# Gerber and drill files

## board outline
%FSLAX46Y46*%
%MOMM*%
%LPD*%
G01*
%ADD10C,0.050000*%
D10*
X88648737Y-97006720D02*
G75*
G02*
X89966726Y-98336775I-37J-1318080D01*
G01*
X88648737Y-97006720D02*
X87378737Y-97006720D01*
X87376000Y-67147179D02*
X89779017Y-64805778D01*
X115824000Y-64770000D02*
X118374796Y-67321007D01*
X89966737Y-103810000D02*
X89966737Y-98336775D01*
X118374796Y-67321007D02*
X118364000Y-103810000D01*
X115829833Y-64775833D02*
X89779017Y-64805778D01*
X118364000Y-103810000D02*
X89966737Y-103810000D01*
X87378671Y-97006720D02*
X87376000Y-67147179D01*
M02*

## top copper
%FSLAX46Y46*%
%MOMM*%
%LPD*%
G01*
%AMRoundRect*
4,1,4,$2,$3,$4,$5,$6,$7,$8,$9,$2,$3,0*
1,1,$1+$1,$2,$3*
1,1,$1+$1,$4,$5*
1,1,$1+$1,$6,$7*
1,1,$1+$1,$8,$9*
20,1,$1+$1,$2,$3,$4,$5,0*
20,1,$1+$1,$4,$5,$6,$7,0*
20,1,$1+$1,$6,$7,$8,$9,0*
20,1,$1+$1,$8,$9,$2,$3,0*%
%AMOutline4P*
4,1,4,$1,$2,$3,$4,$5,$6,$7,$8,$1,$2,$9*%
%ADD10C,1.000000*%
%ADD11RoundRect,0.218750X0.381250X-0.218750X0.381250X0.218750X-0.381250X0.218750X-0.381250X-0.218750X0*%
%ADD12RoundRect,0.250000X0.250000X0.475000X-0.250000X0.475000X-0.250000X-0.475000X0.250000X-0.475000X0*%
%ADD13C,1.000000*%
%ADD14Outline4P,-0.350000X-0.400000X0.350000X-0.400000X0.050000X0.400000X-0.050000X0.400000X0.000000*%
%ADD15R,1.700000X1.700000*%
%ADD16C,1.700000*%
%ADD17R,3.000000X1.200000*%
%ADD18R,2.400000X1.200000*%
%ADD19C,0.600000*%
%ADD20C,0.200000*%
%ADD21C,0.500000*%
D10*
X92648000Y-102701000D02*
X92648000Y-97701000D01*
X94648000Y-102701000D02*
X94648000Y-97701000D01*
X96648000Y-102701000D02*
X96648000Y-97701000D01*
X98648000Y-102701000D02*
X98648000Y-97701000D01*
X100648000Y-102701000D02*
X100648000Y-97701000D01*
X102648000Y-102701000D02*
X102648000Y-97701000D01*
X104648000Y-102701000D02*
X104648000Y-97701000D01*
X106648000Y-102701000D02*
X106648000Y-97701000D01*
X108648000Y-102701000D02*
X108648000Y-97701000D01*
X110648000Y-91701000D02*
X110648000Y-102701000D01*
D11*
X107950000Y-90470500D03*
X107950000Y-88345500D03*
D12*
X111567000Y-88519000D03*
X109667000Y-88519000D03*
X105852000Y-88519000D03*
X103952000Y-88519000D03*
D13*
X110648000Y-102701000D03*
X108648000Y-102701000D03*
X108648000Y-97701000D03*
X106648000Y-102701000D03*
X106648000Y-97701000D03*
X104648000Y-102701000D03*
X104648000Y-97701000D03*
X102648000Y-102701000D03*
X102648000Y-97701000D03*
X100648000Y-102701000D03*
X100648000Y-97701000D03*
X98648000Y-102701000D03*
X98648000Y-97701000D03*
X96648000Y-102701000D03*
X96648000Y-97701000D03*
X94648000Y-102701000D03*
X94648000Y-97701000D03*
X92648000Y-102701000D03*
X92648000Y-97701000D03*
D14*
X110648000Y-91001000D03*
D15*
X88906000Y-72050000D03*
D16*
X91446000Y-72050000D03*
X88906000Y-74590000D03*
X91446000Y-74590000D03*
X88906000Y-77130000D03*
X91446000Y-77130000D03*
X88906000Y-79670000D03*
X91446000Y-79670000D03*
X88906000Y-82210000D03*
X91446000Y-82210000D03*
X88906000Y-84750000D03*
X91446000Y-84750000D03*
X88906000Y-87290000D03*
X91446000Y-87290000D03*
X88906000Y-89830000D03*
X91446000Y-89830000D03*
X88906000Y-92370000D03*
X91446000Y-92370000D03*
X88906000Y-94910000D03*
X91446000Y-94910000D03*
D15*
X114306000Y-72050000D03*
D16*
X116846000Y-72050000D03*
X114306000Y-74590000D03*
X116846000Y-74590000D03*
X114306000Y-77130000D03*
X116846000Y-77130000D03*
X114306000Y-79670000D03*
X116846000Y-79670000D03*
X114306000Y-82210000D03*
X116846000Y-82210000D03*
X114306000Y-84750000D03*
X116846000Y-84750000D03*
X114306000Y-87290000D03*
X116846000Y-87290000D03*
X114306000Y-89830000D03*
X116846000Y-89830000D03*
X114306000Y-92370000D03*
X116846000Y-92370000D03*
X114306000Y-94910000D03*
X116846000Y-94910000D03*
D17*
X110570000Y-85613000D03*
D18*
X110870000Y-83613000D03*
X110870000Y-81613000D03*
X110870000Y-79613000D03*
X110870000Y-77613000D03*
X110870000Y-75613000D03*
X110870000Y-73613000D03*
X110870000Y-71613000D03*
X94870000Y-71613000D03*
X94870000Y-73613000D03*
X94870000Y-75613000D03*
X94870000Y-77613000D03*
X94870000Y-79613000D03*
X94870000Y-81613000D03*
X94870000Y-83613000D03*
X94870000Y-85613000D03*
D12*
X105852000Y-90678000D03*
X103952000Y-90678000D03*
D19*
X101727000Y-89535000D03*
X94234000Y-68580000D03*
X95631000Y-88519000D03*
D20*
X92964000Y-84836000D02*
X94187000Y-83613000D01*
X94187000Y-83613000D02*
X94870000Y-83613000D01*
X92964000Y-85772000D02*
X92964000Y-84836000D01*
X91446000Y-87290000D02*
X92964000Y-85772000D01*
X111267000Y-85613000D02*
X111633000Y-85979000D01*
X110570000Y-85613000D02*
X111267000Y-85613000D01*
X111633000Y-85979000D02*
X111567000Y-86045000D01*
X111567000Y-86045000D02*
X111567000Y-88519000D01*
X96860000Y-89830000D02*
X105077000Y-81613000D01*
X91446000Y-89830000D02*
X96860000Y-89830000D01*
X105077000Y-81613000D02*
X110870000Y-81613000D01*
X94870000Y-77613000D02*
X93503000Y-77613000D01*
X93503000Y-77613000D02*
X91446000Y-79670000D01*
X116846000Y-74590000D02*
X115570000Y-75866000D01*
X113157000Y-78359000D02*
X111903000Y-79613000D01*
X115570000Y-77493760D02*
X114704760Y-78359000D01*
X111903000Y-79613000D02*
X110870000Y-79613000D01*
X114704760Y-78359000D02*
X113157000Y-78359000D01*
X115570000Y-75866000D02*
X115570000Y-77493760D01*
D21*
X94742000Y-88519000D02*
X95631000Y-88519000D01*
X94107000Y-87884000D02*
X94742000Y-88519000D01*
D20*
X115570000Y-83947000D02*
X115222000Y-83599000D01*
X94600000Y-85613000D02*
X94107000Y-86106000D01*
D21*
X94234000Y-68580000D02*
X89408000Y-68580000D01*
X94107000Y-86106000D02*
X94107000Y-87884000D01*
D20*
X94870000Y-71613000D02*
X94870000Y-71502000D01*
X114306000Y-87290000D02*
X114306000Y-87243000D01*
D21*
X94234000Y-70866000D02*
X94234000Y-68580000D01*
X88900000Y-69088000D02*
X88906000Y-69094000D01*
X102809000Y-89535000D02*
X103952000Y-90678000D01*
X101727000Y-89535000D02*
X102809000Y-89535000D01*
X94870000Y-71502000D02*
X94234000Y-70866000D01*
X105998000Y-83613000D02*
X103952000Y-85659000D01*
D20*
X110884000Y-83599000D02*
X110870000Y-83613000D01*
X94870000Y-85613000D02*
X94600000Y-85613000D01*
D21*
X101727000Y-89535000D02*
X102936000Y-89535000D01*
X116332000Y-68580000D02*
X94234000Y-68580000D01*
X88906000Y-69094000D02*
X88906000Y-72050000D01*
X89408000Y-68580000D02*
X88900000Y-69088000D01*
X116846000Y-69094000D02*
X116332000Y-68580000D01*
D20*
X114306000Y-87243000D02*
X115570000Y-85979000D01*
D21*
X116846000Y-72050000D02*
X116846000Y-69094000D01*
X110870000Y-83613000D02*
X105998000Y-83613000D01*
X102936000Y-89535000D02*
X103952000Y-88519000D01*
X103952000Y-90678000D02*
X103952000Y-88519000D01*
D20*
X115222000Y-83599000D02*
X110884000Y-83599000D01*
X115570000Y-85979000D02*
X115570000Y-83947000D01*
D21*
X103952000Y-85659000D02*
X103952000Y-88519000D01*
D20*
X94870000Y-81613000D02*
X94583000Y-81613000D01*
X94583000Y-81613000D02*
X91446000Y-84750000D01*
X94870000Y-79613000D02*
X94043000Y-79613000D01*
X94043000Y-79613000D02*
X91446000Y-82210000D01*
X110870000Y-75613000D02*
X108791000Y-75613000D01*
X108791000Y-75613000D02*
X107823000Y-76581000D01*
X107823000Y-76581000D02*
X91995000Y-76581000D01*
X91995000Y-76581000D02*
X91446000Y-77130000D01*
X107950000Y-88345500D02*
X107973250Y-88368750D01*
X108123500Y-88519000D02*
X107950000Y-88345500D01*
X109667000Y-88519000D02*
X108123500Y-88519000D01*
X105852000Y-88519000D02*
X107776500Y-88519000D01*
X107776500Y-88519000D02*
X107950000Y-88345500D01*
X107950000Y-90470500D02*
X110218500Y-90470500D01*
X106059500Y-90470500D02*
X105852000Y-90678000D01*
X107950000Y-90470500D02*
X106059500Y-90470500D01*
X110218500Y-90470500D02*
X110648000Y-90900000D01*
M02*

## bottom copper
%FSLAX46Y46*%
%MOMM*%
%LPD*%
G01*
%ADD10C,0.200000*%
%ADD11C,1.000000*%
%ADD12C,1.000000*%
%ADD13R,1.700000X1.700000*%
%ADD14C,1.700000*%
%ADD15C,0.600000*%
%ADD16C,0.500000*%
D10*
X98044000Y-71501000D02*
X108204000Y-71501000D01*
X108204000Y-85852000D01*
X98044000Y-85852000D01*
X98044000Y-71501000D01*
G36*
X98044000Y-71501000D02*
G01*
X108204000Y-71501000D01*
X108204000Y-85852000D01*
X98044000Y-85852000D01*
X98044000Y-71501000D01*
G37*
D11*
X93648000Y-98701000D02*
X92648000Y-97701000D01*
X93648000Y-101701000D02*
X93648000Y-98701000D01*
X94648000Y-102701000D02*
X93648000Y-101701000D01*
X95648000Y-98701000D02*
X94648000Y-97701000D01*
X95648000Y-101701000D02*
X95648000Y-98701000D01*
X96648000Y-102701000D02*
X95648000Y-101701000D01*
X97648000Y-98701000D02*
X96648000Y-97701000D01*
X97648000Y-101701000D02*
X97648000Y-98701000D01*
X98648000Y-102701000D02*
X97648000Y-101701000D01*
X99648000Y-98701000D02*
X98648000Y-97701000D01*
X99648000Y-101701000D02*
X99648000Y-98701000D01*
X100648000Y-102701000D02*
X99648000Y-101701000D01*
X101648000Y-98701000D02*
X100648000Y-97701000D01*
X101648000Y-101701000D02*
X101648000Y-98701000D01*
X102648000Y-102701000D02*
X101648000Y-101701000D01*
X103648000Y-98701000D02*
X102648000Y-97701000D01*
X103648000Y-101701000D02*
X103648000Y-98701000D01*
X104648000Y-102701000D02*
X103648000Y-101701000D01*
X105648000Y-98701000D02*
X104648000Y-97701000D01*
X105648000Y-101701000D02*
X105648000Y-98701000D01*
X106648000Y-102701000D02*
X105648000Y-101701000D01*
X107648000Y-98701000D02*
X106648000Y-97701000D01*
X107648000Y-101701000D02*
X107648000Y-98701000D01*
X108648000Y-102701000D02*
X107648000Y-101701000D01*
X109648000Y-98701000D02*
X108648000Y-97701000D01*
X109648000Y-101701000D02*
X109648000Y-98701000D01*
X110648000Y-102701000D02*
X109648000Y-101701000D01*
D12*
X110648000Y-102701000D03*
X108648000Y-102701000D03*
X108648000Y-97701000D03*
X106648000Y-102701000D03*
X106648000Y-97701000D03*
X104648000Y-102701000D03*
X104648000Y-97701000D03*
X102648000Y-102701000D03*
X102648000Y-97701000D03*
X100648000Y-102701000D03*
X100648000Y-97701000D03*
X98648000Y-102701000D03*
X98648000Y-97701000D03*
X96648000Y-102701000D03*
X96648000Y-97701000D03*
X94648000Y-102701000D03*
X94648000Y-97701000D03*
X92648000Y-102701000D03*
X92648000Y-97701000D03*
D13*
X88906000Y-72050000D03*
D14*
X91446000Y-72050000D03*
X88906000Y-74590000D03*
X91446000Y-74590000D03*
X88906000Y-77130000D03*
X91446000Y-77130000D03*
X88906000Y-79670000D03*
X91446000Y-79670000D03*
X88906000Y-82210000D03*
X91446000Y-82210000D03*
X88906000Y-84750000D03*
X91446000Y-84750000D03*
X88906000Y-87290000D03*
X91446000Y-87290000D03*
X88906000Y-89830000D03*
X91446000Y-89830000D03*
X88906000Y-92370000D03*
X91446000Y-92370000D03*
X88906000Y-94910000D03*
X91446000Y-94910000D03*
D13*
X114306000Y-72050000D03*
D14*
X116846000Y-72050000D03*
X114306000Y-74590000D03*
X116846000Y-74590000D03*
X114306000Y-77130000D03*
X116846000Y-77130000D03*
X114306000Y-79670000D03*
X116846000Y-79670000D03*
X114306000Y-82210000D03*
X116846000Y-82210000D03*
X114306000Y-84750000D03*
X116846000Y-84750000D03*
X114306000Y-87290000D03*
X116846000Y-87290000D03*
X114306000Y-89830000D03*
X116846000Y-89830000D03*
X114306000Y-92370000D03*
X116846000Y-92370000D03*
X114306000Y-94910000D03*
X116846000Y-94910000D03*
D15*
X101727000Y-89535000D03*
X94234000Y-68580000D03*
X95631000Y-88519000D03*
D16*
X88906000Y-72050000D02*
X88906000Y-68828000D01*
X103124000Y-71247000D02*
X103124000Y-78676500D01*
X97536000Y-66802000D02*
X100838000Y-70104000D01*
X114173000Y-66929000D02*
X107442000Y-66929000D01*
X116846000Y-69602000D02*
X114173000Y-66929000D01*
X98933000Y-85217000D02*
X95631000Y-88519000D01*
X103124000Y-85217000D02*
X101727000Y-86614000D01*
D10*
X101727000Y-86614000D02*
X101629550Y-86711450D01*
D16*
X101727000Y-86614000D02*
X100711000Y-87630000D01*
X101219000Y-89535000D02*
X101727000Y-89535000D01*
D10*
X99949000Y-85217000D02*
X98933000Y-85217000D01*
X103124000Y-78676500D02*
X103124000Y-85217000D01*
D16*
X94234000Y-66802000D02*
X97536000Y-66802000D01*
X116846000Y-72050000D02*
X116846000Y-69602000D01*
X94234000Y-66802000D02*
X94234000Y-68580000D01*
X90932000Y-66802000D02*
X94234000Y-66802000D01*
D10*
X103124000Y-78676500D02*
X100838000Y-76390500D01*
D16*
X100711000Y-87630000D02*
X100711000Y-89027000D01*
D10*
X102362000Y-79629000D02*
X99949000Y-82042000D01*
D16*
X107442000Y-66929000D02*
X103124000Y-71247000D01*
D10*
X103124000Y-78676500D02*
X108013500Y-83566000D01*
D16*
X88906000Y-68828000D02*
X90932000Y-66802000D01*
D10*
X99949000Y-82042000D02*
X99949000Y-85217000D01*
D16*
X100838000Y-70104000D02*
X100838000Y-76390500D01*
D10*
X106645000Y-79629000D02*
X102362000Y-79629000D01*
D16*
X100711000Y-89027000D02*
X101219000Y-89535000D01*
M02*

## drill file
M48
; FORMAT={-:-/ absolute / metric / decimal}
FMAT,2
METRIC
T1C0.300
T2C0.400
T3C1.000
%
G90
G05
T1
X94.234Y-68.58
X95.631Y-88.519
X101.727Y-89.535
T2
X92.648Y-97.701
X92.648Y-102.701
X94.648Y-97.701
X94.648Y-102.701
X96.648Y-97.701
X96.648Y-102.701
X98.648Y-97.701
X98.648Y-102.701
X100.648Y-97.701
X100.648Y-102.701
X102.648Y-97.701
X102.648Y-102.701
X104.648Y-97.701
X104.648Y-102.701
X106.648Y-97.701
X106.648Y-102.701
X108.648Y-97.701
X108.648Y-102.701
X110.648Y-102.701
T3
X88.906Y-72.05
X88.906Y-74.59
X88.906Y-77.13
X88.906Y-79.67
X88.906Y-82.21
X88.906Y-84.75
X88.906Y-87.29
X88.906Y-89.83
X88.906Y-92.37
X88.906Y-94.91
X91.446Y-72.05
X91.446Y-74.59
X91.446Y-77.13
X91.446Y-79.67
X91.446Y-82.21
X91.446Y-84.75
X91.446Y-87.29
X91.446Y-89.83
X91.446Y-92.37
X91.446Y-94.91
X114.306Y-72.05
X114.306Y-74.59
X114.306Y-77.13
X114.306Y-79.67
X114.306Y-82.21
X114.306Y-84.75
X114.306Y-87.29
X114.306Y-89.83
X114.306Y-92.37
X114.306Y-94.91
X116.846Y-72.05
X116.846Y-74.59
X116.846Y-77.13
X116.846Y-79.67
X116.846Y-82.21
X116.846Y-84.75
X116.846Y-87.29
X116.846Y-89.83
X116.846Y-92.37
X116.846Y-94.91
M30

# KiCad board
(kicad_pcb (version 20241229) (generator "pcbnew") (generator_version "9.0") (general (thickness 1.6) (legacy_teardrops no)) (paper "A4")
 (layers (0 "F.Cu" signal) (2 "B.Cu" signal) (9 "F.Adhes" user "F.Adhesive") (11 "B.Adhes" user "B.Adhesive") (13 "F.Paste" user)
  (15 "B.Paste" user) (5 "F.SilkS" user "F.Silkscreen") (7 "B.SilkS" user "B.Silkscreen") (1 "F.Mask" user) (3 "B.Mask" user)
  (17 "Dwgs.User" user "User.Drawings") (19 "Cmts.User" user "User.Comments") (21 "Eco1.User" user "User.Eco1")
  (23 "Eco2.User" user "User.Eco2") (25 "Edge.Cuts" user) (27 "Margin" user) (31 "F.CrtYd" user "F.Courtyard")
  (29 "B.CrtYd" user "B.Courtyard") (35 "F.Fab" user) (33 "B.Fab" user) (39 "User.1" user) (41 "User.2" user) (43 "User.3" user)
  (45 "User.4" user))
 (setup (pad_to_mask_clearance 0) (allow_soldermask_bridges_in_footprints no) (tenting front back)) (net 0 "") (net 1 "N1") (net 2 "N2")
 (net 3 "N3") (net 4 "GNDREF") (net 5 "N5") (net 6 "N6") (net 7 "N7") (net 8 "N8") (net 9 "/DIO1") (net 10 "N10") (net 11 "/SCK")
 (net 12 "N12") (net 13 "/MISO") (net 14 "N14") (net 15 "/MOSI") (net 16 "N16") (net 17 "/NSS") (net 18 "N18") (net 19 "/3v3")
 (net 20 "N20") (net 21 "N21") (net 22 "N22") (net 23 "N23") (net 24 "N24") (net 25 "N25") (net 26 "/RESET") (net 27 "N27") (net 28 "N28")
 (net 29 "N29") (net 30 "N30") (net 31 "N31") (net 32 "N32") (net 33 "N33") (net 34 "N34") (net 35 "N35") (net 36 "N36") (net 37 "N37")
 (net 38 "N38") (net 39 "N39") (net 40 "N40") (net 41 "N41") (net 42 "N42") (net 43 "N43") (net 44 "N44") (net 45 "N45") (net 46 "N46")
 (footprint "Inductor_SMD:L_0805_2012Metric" (layer "F.Cu") (at 107.95 89.408 90)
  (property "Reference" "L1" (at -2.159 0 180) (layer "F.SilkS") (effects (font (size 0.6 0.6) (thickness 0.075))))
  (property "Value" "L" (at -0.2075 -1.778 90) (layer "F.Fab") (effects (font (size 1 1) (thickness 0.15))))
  (pad "1" smd roundrect (at -1.0625 0 90) (size 0.875 1.2) (layers "F.Cu" "F.Mask" "F.Paste") (roundrect_rratio 0.25) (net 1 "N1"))
  (pad "2" smd roundrect (at 1.0625 0 90) (size 0.875 1.2) (layers "F.Cu" "F.Mask" "F.Paste") (roundrect_rratio 0.25) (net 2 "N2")))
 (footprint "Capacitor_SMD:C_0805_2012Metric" (layer "F.Cu") (at 110.617 88.519 180)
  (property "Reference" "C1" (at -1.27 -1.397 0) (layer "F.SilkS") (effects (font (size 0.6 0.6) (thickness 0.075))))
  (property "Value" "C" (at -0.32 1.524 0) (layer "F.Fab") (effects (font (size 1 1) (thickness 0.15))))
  (pad "1" smd roundrect (at -0.95 0 180) (size 1 1.45) (layers "F.Cu" "F.Mask" "F.Paste") (roundrect_rratio 0.25) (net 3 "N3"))
  (pad "2" smd roundrect (at 0.95 0 180) (size 1 1.45) (layers "F.Cu" "F.Mask" "F.Paste") (roundrect_rratio 0.25) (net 2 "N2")))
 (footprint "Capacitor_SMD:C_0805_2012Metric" (layer "F.Cu") (at 104.902 88.519 180)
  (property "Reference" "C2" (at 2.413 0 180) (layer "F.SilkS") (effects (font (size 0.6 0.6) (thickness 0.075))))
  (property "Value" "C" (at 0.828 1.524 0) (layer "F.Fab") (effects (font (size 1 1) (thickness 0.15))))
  (pad "1" smd roundrect (at -0.95 0 180) (size 1 1.45) (layers "F.Cu" "F.Mask" "F.Paste") (roundrect_rratio 0.25) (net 2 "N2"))
  (pad "2" smd roundrect (at 0.95 0 180) (size 1 1.45) (layers "F.Cu" "F.Mask" "F.Paste") (roundrect_rratio 0.25) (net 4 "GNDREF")))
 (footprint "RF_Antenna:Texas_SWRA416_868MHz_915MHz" (layer "F.Cu") (at 101.648 96.901 180)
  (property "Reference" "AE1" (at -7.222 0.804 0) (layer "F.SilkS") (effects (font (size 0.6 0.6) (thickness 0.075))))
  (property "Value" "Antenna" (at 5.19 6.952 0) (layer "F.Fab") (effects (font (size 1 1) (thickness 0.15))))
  (fp_line (start 9 -5.8) (end 9 -0.8) (stroke (width 1) (type solid)) (layer "F.Cu"))
  (fp_line (start 7 -5.8) (end 7 -0.8) (stroke (width 1) (type solid)) (layer "F.Cu"))
  (fp_line (start 5 -5.8) (end 5 -0.8) (stroke (width 1) (type solid)) (layer "F.Cu"))
  (fp_line (start 3 -5.8) (end 3 -0.8) (stroke (width 1) (type solid)) (layer "F.Cu"))
  (fp_line (start 1 -5.8) (end 1 -0.8) (stroke (width 1) (type solid)) (layer "F.Cu"))
  (fp_line (start -1 -5.8) (end -1 -0.8) (stroke (width 1) (type solid)) (layer "F.Cu"))
  (fp_line (start -3 -5.8) (end -3 -0.8) (stroke (width 1) (type solid)) (layer "F.Cu"))
  (fp_line (start -5 -5.8) (end -5 -0.8) (stroke (width 1) (type solid)) (layer "F.Cu"))
  (fp_line (start -7 -5.8) (end -7 -0.8) (stroke (width 1) (type solid)) (layer "F.Cu"))
  (fp_line (start -9 5.2) (end -9 -5.8) (stroke (width 1) (type solid)) (layer "F.Cu"))
  (fp_line (start 8 -1.8) (end 9 -0.8) (stroke (width 1) (type solid)) (layer "B.Cu"))
  (fp_line (start 8 -4.8) (end 8 -1.8) (stroke (width 1) (type solid)) (layer "B.Cu"))
  (fp_line (start 7 -5.8) (end 8 -4.8) (stroke (width 1) (type solid)) (layer "B.Cu"))
  (fp_line (start 6 -1.8) (end 7 -0.8) (stroke (width 1) (type solid)) (layer "B.Cu"))
  (fp_line (start 6 -4.8) (end 6 -1.8) (stroke (width 1) (type solid)) (layer "B.Cu"))
  (fp_line (start 5 -5.8) (end 6 -4.8) (stroke (width 1) (type solid)) (layer "B.Cu"))
  (fp_line (start 4 -1.8) (end 5 -0.8) (stroke (width 1) (type solid)) (layer "B.Cu"))
  (fp_line (start 4 -4.8) (end 4 -1.8) (stroke (width 1) (type solid)) (layer "B.Cu"))
  (fp_line (start 3 -5.8) (end 4 -4.8) (stroke (width 1) (type solid)) (layer "B.Cu"))
  (fp_line (start 2 -1.8) (end 3 -0.8) (stroke (width 1) (type solid)) (layer "B.Cu"))
  (fp_line (start 2 -4.8) (end 2 -1.8) (stroke (width 1) (type solid)) (layer "B.Cu"))
  (fp_line (start 1 -5.8) (end 2 -4.8) (stroke (width 1) (type solid)) (layer "B.Cu"))
  (fp_line (start 0 -1.8) (end 1 -0.8) (stroke (width 1) (type solid)) (layer "B.Cu"))
  (fp_line (start 0 -4.8) (end 0 -1.8) (stroke (width 1) (type solid)) (layer "B.Cu"))
  (fp_line (start -1 -5.8) (end 0 -4.8) (stroke (width 1) (type solid)) (layer "B.Cu"))
  (fp_line (start -2 -1.8) (end -1 -0.8) (stroke (width 1) (type solid)) (layer "B.Cu"))
  (fp_line (start -2 -4.8) (end -2 -1.8) (stroke (width 1) (type solid)) (layer "B.Cu"))
  (fp_line (start -3 -5.8) (end -2 -4.8) (stroke (width 1) (type solid)) (layer "B.Cu"))
  (fp_line (start -4 -1.8) (end -3 -0.8) (stroke (width 1) (type solid)) (layer "B.Cu"))
  (fp_line (start -4 -4.8) (end -4 -1.8) (stroke (width 1) (type solid)) (layer "B.Cu"))
  (fp_line (start -5 -5.8) (end -4 -4.8) (stroke (width 1) (type solid)) (layer "B.Cu"))
  (fp_line (start -6 -1.8) (end -5 -0.8) (stroke (width 1) (type solid)) (layer "B.Cu"))
  (fp_line (start -6 -4.8) (end -6 -1.8) (stroke (width 1) (type solid)) (layer "B.Cu"))
  (fp_line (start -7 -5.8) (end -6 -4.8) (stroke (width 1) (type solid)) (layer "B.Cu"))
  (fp_line (start -8 -1.8) (end -7 -0.8) (stroke (width 1) (type solid)) (layer "B.Cu"))
  (fp_line (start -8 -4.8) (end -8 -1.8) (stroke (width 1) (type solid)) (layer "B.Cu"))
  (fp_line (start -9 -5.8) (end -8 -4.8) (stroke (width 1) (type solid)) (layer "B.Cu"))
  (pad "" thru_hole circle (at -9 -5.8) (size 1 1) (drill 0.4) (layers "*.Cu") (remove_unused_layers no))
  (pad "" thru_hole circle (at -7 -5.8) (size 1 1) (drill 0.4) (layers "*.Cu") (remove_unused_layers no))
  (pad "" thru_hole circle (at -7 -0.8) (size 1 1) (drill 0.4) (layers "*.Cu") (remove_unused_layers no))
  (pad "" thru_hole circle (at -5 -5.8) (size 1 1) (drill 0.4) (layers "*.Cu") (remove_unused_layers no))
  (pad "" thru_hole circle (at -5 -0.8) (size 1 1) (drill 0.4) (layers "*.Cu") (remove_unused_layers no))
  (pad "" thru_hole circle (at -3 -5.8) (size 1 1) (drill 0.4) (layers "*.Cu") (remove_unused_layers no))
  (pad "" thru_hole circle (at -3 -0.8) (size 1 1) (drill 0.4) (layers "*.Cu") (remove_unused_layers no))
  (pad "" thru_hole circle (at -1 -5.8) (size 1 1) (drill 0.4) (layers "*.Cu") (remove_unused_layers no))
  (pad "" thru_hole circle (at -1 -0.8) (size 1 1) (drill 0.4) (layers "*.Cu") (remove_unused_layers no))
  (pad "" thru_hole circle (at 1 -5.8) (size 1 1) (drill 0.4) (layers "*.Cu") (remove_unused_layers no))
  (pad "" thru_hole circle (at 1 -0.8) (size 1 1) (drill 0.4) (layers "*.Cu") (remove_unused_layers no))
  (pad "" thru_hole circle (at 3 -5.8) (size 1 1) (drill 0.4) (layers "*.Cu") (remove_unused_layers no))
  (pad "" thru_hole circle (at 3 -0.8) (size 1 1) (drill 0.4) (layers "*.Cu") (remove_unused_layers no))
  (pad "" thru_hole circle (at 5 -5.8) (size 1 1) (drill 0.4) (layers "*.Cu") (remove_unused_layers no))
  (pad "" thru_hole circle (at 5 -0.8) (size 1 1) (drill 0.4) (layers "*.Cu") (remove_unused_layers no))
  (pad "" thru_hole circle (at 7 -5.8) (size 1 1) (drill 0.4) (layers "*.Cu") (remove_unused_layers no))
  (pad "" thru_hole circle (at 7 -0.8) (size 1 1) (drill 0.4) (layers "*.Cu") (remove_unused_layers no))
  (pad "" thru_hole circle (at 9 -5.8) (size 1 1) (drill 0.4) (layers "*.Cu") (remove_unused_layers no))
  (pad "" thru_hole circle (at 9 -0.8) (size 1 1) (drill 0.4) (layers "*.Cu") (remove_unused_layers no))
  (pad "1" smd trapezoid (at -9 5.9) (size 0.4 0.8) (rect_delta 0 0.3) (layers "F.Cu") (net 1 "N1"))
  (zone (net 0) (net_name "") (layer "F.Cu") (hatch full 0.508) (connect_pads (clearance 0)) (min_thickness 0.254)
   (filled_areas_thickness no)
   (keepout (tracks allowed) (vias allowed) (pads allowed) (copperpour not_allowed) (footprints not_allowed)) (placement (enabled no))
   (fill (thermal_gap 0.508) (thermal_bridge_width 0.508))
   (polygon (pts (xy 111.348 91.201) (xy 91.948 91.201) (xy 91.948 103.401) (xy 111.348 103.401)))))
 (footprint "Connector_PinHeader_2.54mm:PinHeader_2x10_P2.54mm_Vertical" (layer "F.Cu") (at 88.906 72.05)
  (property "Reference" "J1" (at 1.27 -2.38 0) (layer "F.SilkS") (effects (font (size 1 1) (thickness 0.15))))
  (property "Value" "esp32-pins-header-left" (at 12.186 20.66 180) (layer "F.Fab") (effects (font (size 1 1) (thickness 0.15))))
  (pad "1" thru_hole rect (at 0 0) (size 1.7 1.7) (drill 1) (layers "*.Cu" "*.Mask") (remove_unused_layers no) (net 4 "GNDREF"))
  (pad "2" thru_hole circle (at 2.54 0) (size 1.7 1.7) (drill 1) (layers "*.Cu" "*.Mask") (remove_unused_layers no) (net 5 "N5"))
  (pad "3" thru_hole circle (at 0 2.54) (size 1.7 1.7) (drill 1) (layers "*.Cu" "*.Mask") (remove_unused_layers no) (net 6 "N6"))
  (pad "4" thru_hole circle (at 2.54 2.54) (size 1.7 1.7) (drill 1) (layers "*.Cu" "*.Mask") (remove_unused_layers no) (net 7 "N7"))
  (pad "5" thru_hole circle (at 0 5.08) (size 1.7 1.7) (drill 1) (layers "*.Cu" "*.Mask") (remove_unused_layers no) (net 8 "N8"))
  (pad "6" thru_hole circle (at 2.54 5.08) (size 1.7 1.7) (drill 1) (layers "*.Cu" "*.Mask") (remove_unused_layers no) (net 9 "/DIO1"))
  (pad "7" thru_hole circle (at 0 7.62) (size 1.7 1.7) (drill 1) (layers "*.Cu" "*.Mask") (remove_unused_layers no) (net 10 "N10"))
  (pad "8" thru_hole circle (at 2.54 7.62) (size 1.7 1.7) (drill 1) (layers "*.Cu" "*.Mask") (remove_unused_layers no) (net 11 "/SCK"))
  (pad "9" thru_hole circle (at 0 10.16) (size 1.7 1.7) (drill 1) (layers "*.Cu" "*.Mask") (remove_unused_layers no) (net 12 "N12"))
  (pad "10" thru_hole circle (at 2.54 10.16) (size 1.7 1.7) (drill 1) (layers "*.Cu" "*.Mask") (remove_unused_layers no) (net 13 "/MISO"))
  (pad "11" thru_hole circle (at 0 12.7) (size 1.7 1.7) (drill 1) (layers "*.Cu" "*.Mask") (remove_unused_layers no) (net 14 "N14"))
  (pad "12" thru_hole circle (at 2.54 12.7) (size 1.7 1.7) (drill 1) (layers "*.Cu" "*.Mask") (remove_unused_layers no) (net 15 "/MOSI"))
  (pad "13" thru_hole circle (at 0 15.24) (size 1.7 1.7) (drill 1) (layers "*.Cu" "*.Mask") (remove_unused_layers no) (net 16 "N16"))
  (pad "14" thru_hole circle (at 2.54 15.24) (size 1.7 1.7) (drill 1) (layers "*.Cu" "*.Mask") (remove_unused_layers no) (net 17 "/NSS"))
  (pad "15" thru_hole circle (at 0 17.78) (size 1.7 1.7) (drill 1) (layers "*.Cu" "*.Mask") (remove_unused_layers no) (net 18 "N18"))
  (pad "16" thru_hole circle (at 2.54 17.78) (size 1.7 1.7) (drill 1) (layers "*.Cu" "*.Mask") (remove_unused_layers no) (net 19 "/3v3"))
  (pad "17" thru_hole circle (at 0 20.32) (size 1.7 1.7) (drill 1) (layers "*.Cu" "*.Mask") (remove_unused_layers no) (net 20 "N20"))
  (pad "18" thru_hole circle (at 2.54 20.32) (size 1.7 1.7) (drill 1) (layers "*.Cu" "*.Mask") (remove_unused_layers no) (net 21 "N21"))
  (pad "19" thru_hole circle (at 0 22.86) (size 1.7 1.7) (drill 1) (layers "*.Cu" "*.Mask") (remove_unused_layers no) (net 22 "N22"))
  (pad "20" thru_hole circle (at 2.54 22.86) (size 1.7 1.7) (drill 1) (layers "*.Cu" "*.Mask") (remove_unused_layers no) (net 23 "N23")))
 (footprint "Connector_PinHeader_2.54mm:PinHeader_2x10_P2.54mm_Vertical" (layer "F.Cu") (at 114.306 72.05)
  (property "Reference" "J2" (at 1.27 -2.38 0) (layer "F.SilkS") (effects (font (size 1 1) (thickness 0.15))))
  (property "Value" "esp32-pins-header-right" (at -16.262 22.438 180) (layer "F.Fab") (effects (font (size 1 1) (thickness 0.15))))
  (pad "1" thru_hole rect (at 0 0) (size 1.7 1.7) (drill 1) (layers "*.Cu" "*.Mask") (remove_unused_layers no) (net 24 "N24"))
  (pad "2" thru_hole circle (at 2.54 0) (size 1.7 1.7) (drill 1) (layers "*.Cu" "*.Mask") (remove_unused_layers no) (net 4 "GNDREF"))
  (pad "3" thru_hole circle (at 0 2.54) (size 1.7 1.7) (drill 1) (layers "*.Cu" "*.Mask") (remove_unused_layers no) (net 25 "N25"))
  (pad "4" thru_hole circle (at 2.54 2.54) (size 1.7 1.7) (drill 1) (layers "*.Cu" "*.Mask") (remove_unused_layers no) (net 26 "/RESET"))
  (pad "5" thru_hole circle (at 0 5.08) (size 1.7 1.7) (drill 1) (layers "*.Cu" "*.Mask") (remove_unused_layers no) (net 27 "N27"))
  (pad "6" thru_hole circle (at 2.54 5.08) (size 1.7 1.7) (drill 1) (layers "*.Cu" "*.Mask") (remove_unused_layers no) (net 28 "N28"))
  (pad "7" thru_hole circle (at 0 7.62) (size 1.7 1.7) (drill 1) (layers "*.Cu" "*.Mask") (remove_unused_layers no) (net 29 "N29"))
  (pad "8" thru_hole circle (at 2.54 7.62) (size 1.7 1.7) (drill 1) (layers "*.Cu" "*.Mask") (remove_unused_layers no) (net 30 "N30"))
  (pad "9" thru_hole circle (at 0 10.16) (size 1.7 1.7) (drill 1) (layers "*.Cu" "*.Mask") (remove_unused_layers no) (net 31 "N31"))
  (pad "10" thru_hole circle (at 2.54 10.16) (size 1.7 1.7) (drill 1) (layers "*.Cu" "*.Mask") (remove_unused_layers no) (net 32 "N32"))
  (pad "11" thru_hole circle (at 0 12.7) (size 1.7 1.7) (drill 1) (layers "*.Cu" "*.Mask") (remove_unused_layers no) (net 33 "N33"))
  (pad "12" thru_hole circle (at 2.54 12.7) (size 1.7 1.7) (drill 1) (layers "*.Cu" "*.Mask") (remove_unused_layers no) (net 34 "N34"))
  (pad "13" thru_hole circle (at 0 15.24) (size 1.7 1.7) (drill 1) (layers "*.Cu" "*.Mask") (remove_unused_layers no) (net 4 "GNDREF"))
  (pad "14" thru_hole circle (at 2.54 15.24) (size 1.7 1.7) (drill 1) (layers "*.Cu" "*.Mask") (remove_unused_layers no) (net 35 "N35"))
  (pad "15" thru_hole circle (at 0 17.78) (size 1.7 1.7) (drill 1) (layers "*.Cu" "*.Mask") (remove_unused_layers no) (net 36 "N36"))
  (pad "16" thru_hole circle (at 2.54 17.78) (size 1.7 1.7) (drill 1) (layers "*.Cu" "*.Mask") (remove_unused_layers no) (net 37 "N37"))
  (pad "17" thru_hole circle (at 0 20.32) (size 1.7 1.7) (drill 1) (layers "*.Cu" "*.Mask") (remove_unused_layers no) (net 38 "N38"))
  (pad "18" thru_hole circle (at 2.54 20.32) (size 1.7 1.7) (drill 1) (layers "*.Cu" "*.Mask") (remove_unused_layers no) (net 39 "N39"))
  (pad "19" thru_hole circle (at 0 22.86) (size 1.7 1.7) (drill 1) (layers "*.Cu" "*.Mask") (remove_unused_layers no) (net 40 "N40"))
  (pad "20" thru_hole circle (at 2.54 22.86) (size 1.7 1.7) (drill 1) (layers "*.Cu" "*.Mask") (remove_unused_layers no) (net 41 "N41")))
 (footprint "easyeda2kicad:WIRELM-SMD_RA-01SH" (layer "F.Cu") (at 102.87 78.613 180)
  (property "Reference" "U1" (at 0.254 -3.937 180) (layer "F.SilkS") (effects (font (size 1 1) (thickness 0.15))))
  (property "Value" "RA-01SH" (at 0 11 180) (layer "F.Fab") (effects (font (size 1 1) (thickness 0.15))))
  (pad "1" smd rect (at -7.7 -7 180) (size 3 1.2) (layers "F.Cu" "F.Mask" "F.Paste") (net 3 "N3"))
  (pad "2" smd rect (at -8 -5 180) (size 2.4 1.2) (layers "F.Cu" "F.Mask" "F.Paste") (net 4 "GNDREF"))
  (pad "3" smd rect (at -8 -3 180) (size 2.4 1.2) (layers "F.Cu" "F.Mask" "F.Paste") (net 19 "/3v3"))
  (pad "4" smd rect (at -8 -1 180) (size 2.4 1.2) (layers "F.Cu" "F.Mask" "F.Paste") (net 26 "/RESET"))
  (pad "5" smd rect (at -8 1 180) (size 2.4 1.2) (layers "F.Cu" "F.Mask" "F.Paste") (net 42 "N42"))
  (pad "6" smd rect (at -8 3 180) (size 2.4 1.2) (layers "F.Cu" "F.Mask" "F.Paste") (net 9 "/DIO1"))
  (pad "7" smd rect (at -8 5 180) (size 2.4 1.2) (layers "F.Cu" "F.Mask" "F.Paste") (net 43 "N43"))
  (pad "8" smd rect (at -8 7 180) (size 2.4 1.2) (layers "F.Cu" "F.Mask" "F.Paste") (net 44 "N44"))
  (pad "9" smd rect (at 8 7 180) (size 2.4 1.2) (layers "F.Cu" "F.Mask" "F.Paste") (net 4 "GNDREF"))
  (pad "10" smd rect (at 8 5 180) (size 2.4 1.2) (layers "F.Cu" "F.Mask" "F.Paste") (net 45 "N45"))
  (pad "11" smd rect (at 8 3 180) (size 2.4 1.2) (layers "F.Cu" "F.Mask" "F.Paste") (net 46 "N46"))
  (pad "12" smd rect (at 8 1 180) (size 2.4 1.2) (layers "F.Cu" "F.Mask" "F.Paste") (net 11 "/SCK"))
  (pad "13" smd rect (at 8 -1 180) (size 2.4 1.2) (layers "F.Cu" "F.Mask" "F.Paste") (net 13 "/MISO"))
  (pad "14" smd rect (at 8 -3 180) (size 2.4 1.2) (layers "F.Cu" "F.Mask" "F.Paste") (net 15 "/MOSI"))
  (pad "15" smd rect (at 8 -5 180) (size 2.4 1.2) (layers "F.Cu" "F.Mask" "F.Paste") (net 17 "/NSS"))
  (pad "16" smd rect (at 8 -7 180) (size 2.4 1.2) (layers "F.Cu" "F.Mask" "F.Paste") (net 4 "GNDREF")))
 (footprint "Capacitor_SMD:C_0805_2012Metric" (layer "F.Cu") (at 104.902 90.678 180)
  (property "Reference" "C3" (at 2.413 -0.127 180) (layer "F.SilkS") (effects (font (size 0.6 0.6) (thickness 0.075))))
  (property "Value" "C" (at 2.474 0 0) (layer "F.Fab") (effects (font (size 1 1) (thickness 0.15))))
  (pad "1" smd roundrect (at -0.95 0 180) (size 1 1.45) (layers "F.Cu" "F.Mask" "F.Paste") (roundrect_rratio 0.25) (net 1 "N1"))
  (pad "2" smd roundrect (at 0.95 0 180) (size 1 1.45) (layers "F.Cu" "F.Mask" "F.Paste") (roundrect_rratio 0.25) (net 4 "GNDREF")))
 (gr_rect (start 98.044 71.501) (end 108.204 85.852) (stroke (width 0.2) (type solid)) (fill yes) (layer "B.Cu") (net 4))
 (gr_arc (start 88.648737 97.00672) (mid 89.584975 97.397022) (end 89.966737 98.336775) (stroke (width 0.05) (type default))
  (layer "Edge.Cuts"))
 (gr_line (start 88.648737 97.00672) (end 87.378737 97.00672) (stroke (width 0.05) (type default)) (layer "Edge.Cuts"))
 (gr_line (start 87.376 67.147179) (end 89.779017 64.805778) (stroke (width 0.05) (type default)) (layer "Edge.Cuts"))
 (gr_line (start 115.824 64.77) (end 118.374796 67.321007) (stroke (width 0.05) (type default)) (layer "Edge.Cuts"))
 (gr_line (start 89.966737 103.81) (end 89.966737 98.336775) (stroke (width 0.05) (type default)) (layer "Edge.Cuts"))
 (gr_line (start 118.374796 67.321007) (end 118.364 103.81) (stroke (width 0.05) (type default)) (layer "Edge.Cuts"))
 (gr_line (start 115.829833 64.775833) (end 89.779017 64.805778) (stroke (width 0.05) (type default)) (layer "Edge.Cuts"))
 (gr_line (start 118.364 103.81) (end 89.966737 103.81) (stroke (width 0.05) (type default)) (layer "Edge.Cuts"))
 (gr_line (start 87.378671 97.00672) (end 87.376 67.147179) (stroke (width 0.05) (type default)) (layer "Edge.Cuts"))
 (segment (start 111.267 85.613) (end 111.633 85.979) (width 0.2) (layer "F.Cu") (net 3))
 (segment (start 110.57 85.613) (end 111.267 85.613) (width 0.2) (layer "F.Cu") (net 3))
 (segment (start 111.633 85.979) (end 111.567 86.045) (width 0.2) (layer "F.Cu") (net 3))
 (segment (start 111.567 86.045) (end 111.567 88.519) (width 0.2) (layer "F.Cu") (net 3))
 (segment (start 94.742 88.519) (end 95.631 88.519) (width 0.5) (layer "F.Cu") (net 4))
 (segment (start 94.107 87.884) (end 94.742 88.519) (width 0.5) (layer "F.Cu") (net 4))
 (segment (start 115.57 83.947) (end 115.222 83.599) (width 0.2) (layer "F.Cu") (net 4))
 (segment (start 94.6 85.613) (end 94.107 86.106) (width 0.2) (layer "F.Cu") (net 4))
 (segment (start 94.234 68.58) (end 89.408 68.58) (width 0.5) (layer "F.Cu") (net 4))
 (segment (start 94.107 86.106) (end 94.107 87.884) (width 0.5) (layer "F.Cu") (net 4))
 (segment (start 94.87 71.613) (end 94.87 71.502) (width 0.2) (layer "F.Cu") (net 4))
 (segment (start 114.306 87.29) (end 114.306 87.243) (width 0.2) (layer "F.Cu") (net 4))
 (segment (start 94.234 70.866) (end 94.234 68.58) (width 0.5) (layer "F.Cu") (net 4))
 (segment (start 88.9 69.088) (end 88.906 69.094) (width 0.5) (layer "F.Cu") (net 4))
 (segment (start 102.809 89.535) (end 103.952 90.678) (width 0.5) (layer "F.Cu") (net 4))
 (segment (start 101.727 89.535) (end 102.809 89.535) (width 0.5) (layer "F.Cu") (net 4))
 (segment (start 94.87 71.502) (end 94.234 70.866) (width 0.5) (layer "F.Cu") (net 4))
 (segment (start 105.998 83.613) (end 103.952 85.659) (width 0.5) (layer "F.Cu") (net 4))
 (segment (start 110.884 83.599) (end 110.87 83.613) (width 0.2) (layer "F.Cu") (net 4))
 (segment (start 94.87 85.613) (end 94.6 85.613) (width 0.2) (layer "F.Cu") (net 4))
 (segment (start 101.727 89.535) (end 102.936 89.535) (width 0.5) (layer "F.Cu") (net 4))
 (segment (start 116.332 68.58) (end 94.234 68.58) (width 0.5) (layer "F.Cu") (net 4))
 (segment (start 88.906 69.094) (end 88.906 72.05) (width 0.5) (layer "F.Cu") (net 4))
 (segment (start 89.408 68.58) (end 88.9 69.088) (width 0.5) (layer "F.Cu") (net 4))
 (segment (start 116.846 69.094) (end 116.332 68.58) (width 0.5) (layer "F.Cu") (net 4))
 (segment (start 114.306 87.243) (end 115.57 85.979) (width 0.2) (layer "F.Cu") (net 4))
 (segment (start 116.846 72.05) (end 116.846 69.094) (width 0.5) (layer "F.Cu") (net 4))
 (segment (start 110.87 83.613) (end 105.998 83.613) (width 0.5) (layer "F.Cu") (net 4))
 (segment (start 102.936 89.535) (end 103.952 88.519) (width 0.5) (layer "F.Cu") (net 4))
 (segment (start 103.952 90.678) (end 103.952 88.519) (width 0.5) (layer "F.Cu") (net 4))
 (segment (start 115.222 83.599) (end 110.884 83.599) (width 0.2) (layer "F.Cu") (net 4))
 (segment (start 115.57 85.979) (end 115.57 83.947) (width 0.2) (layer "F.Cu") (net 4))
 (segment (start 103.952 85.659) (end 103.952 88.519) (width 0.5) (layer "F.Cu") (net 4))
 (via (at 101.727 89.535) (size 0.6) (drill 0.3) (layers "F.Cu" "B.Cu") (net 4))
 (via (at 94.234 68.58) (size 0.6) (drill 0.3) (layers "F.Cu" "B.Cu") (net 4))
 (via (at 95.631 88.519) (size 0.6) (drill 0.3) (layers "F.Cu" "B.Cu") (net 4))
 (segment (start 88.906 72.05) (end 88.906 68.828) (width 0.5) (layer "B.Cu") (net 4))
 (segment (start 103.124 71.247) (end 103.124 78.6765) (width 0.5) (layer "B.Cu") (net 4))
 (segment (start 97.536 66.802) (end 100.838 70.104) (width 0.5) (layer "B.Cu") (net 4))
 (segment (start 114.173 66.929) (end 107.442 66.929) (width 0.5) (layer "B.Cu") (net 4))
 (segment (start 116.846 69.602) (end 114.173 66.929) (width 0.5) (layer "B.Cu") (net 4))
 (segment (start 98.933 85.217) (end 95.631 88.519) (width 0.5) (layer "B.Cu") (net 4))
 (segment (start 103.124 85.217) (end 101.727 86.614) (width 0.5) (layer "B.Cu") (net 4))
 (segment (start 101.727 86.614) (end 101.62955 86.71145) (width 0.2) (layer "B.Cu") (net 4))
 (segment (start 101.727 86.614) (end 100.711 87.63) (width 0.5) (layer "B.Cu") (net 4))
 (segment (start 101.219 89.535) (end 101.727 89.535) (width 0.5) (layer "B.Cu") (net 4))
 (segment (start 99.949 85.217) (end 98.933 85.217) (width 0.2) (layer "B.Cu") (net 4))
 (segment (start 103.124 78.6765) (end 103.124 85.217) (width 0.2) (layer "B.Cu") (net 4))
 (segment (start 94.234 66.802) (end 97.536 66.802) (width 0.5) (layer "B.Cu") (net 4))
 (segment (start 116.846 72.05) (end 116.846 69.602) (width 0.5) (layer "B.Cu") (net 4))
 (segment (start 94.234 66.802) (end 94.234 68.58) (width 0.5) (layer "B.Cu") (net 4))
 (segment (start 90.932 66.802) (end 94.234 66.802) (width 0.5) (layer "B.Cu") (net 4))
 (segment (start 103.124 78.6765) (end 100.838 76.3905) (width 0.2) (layer "B.Cu") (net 4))
 (segment (start 100.711 87.63) (end 100.711 89.027) (width 0.5) (layer "B.Cu") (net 4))
 (segment (start 102.362 79.629) (end 99.949 82.042) (width 0.2) (layer "B.Cu") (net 4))
 (segment (start 107.442 66.929) (end 103.124 71.247) (width 0.5) (layer "B.Cu") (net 4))
 (segment (start 103.124 78.6765) (end 108.0135 83.566) (width 0.2) (layer "B.Cu") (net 4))
 (segment (start 88.906 68.828) (end 90.932 66.802) (width 0.5) (layer "B.Cu") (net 4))
 (segment (start 99.949 82.042) (end 99.949 85.217) (width 0.2) (layer "B.Cu") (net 4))
 (segment (start 100.838 70.104) (end 100.838 76.3905) (width 0.5) (layer "B.Cu") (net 4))
 (segment (start 106.645 79.629) (end 102.362 79.629) (width 0.2) (layer "B.Cu") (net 4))
 (segment (start 100.711 89.027) (end 101.219 89.535) (width 0.5) (layer "B.Cu") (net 4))
 (segment (start 94.87 81.613) (end 94.583 81.613) (width 0.2) (layer "F.Cu") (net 15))
 (segment (start 94.583 81.613) (end 91.446 84.75) (width 0.2) (layer "F.Cu") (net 15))
 (segment (start 94.87 77.613) (end 93.503 77.613) (width 0.2) (layer "F.Cu") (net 11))
 (segment (start 93.503 77.613) (end 91.446 79.67) (width 0.2) (layer "F.Cu") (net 11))
 (segment (start 92.964 84.836) (end 94.187 83.613) (width 0.2) (layer "F.Cu") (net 17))
 (segment (start 94.187 83.613) (end 94.87 83.613) (width 0.2) (layer "F.Cu") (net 17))
 (segment (start 92.964 85.772) (end 92.964 84.836) (width 0.2) (layer "F.Cu") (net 17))
 (segment (start 91.446 87.29) (end 92.964 85.772) (width 0.2) (layer "F.Cu") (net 17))
 (segment (start 107.95 88.3455) (end 107.97325 88.36875) (width 0.2) (layer "F.Cu") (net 2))
 (segment (start 108.1235 88.519) (end 107.95 88.3455) (width 0.2) (layer "F.Cu") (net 2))
 (segment (start 109.667 88.519) (end 108.1235 88.519) (width 0.2) (layer "F.Cu") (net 2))
 (segment (start 105.852 88.519) (end 107.7765 88.519) (width 0.2) (layer "F.Cu") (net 2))
 (segment (start 107.7765 88.519) (end 107.95 88.3455) (width 0.2) (layer "F.Cu") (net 2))
 (segment (start 107.95 90.4705) (end 110.2185 90.4705) (width 0.2) (layer "F.Cu") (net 1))
 (segment (start 106.0595 90.4705) (end 105.852 90.678) (width 0.2) (layer "F.Cu") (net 1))
 (segment (start 107.95 90.4705) (end 106.0595 90.4705) (width 0.2) (layer "F.Cu") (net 1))
 (segment (start 110.2185 90.4705) (end 110.648 90.9) (width 0.2) (layer "F.Cu") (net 1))
 (segment (start 110.87 75.613) (end 108.791 75.613) (width 0.2) (layer "F.Cu") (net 9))
 (segment (start 108.791 75.613) (end 107.823 76.581) (width 0.2) (layer "F.Cu") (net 9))
 (segment (start 107.823 76.581) (end 91.995 76.581) (width 0.2) (layer "F.Cu") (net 9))
 (segment (start 91.995 76.581) (end 91.446 77.13) (width 0.2) (layer "F.Cu") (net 9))
 (segment (start 94.87 79.613) (end 94.043 79.613) (width 0.2) (layer "F.Cu") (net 13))
 (segment (start 94.043 79.613) (end 91.446 82.21) (width 0.2) (layer "F.Cu") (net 13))
 (segment (start 96.86 89.83) (end 105.077 81.613) (width 0.2) (layer "F.Cu") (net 19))
 (segment (start 91.446 89.83) (end 96.86 89.83) (width 0.2) (layer "F.Cu") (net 19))
 (segment (start 105.077 81.613) (end 110.87 81.613) (width 0.2) (layer "F.Cu") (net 19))
 (segment (start 116.846 74.59) (end 115.57 75.866) (width 0.2) (layer "F.Cu") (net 26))
 (segment (start 113.157 78.359) (end 111.903 79.613) (width 0.2) (layer "F.Cu") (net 26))
 (segment (start 115.57 77.49376) (end 114.70476 78.359) (width 0.2) (layer "F.Cu") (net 26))
 (segment (start 111.903 79.613) (end 110.87 79.613) (width 0.2) (layer "F.Cu") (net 26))
 (segment (start 114.70476 78.359) (end 113.157 78.359) (width 0.2) (layer "F.Cu") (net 26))
 (segment (start 115.57 75.866) (end 115.57 77.49376) (width 0.2) (layer "F.Cu") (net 26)))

